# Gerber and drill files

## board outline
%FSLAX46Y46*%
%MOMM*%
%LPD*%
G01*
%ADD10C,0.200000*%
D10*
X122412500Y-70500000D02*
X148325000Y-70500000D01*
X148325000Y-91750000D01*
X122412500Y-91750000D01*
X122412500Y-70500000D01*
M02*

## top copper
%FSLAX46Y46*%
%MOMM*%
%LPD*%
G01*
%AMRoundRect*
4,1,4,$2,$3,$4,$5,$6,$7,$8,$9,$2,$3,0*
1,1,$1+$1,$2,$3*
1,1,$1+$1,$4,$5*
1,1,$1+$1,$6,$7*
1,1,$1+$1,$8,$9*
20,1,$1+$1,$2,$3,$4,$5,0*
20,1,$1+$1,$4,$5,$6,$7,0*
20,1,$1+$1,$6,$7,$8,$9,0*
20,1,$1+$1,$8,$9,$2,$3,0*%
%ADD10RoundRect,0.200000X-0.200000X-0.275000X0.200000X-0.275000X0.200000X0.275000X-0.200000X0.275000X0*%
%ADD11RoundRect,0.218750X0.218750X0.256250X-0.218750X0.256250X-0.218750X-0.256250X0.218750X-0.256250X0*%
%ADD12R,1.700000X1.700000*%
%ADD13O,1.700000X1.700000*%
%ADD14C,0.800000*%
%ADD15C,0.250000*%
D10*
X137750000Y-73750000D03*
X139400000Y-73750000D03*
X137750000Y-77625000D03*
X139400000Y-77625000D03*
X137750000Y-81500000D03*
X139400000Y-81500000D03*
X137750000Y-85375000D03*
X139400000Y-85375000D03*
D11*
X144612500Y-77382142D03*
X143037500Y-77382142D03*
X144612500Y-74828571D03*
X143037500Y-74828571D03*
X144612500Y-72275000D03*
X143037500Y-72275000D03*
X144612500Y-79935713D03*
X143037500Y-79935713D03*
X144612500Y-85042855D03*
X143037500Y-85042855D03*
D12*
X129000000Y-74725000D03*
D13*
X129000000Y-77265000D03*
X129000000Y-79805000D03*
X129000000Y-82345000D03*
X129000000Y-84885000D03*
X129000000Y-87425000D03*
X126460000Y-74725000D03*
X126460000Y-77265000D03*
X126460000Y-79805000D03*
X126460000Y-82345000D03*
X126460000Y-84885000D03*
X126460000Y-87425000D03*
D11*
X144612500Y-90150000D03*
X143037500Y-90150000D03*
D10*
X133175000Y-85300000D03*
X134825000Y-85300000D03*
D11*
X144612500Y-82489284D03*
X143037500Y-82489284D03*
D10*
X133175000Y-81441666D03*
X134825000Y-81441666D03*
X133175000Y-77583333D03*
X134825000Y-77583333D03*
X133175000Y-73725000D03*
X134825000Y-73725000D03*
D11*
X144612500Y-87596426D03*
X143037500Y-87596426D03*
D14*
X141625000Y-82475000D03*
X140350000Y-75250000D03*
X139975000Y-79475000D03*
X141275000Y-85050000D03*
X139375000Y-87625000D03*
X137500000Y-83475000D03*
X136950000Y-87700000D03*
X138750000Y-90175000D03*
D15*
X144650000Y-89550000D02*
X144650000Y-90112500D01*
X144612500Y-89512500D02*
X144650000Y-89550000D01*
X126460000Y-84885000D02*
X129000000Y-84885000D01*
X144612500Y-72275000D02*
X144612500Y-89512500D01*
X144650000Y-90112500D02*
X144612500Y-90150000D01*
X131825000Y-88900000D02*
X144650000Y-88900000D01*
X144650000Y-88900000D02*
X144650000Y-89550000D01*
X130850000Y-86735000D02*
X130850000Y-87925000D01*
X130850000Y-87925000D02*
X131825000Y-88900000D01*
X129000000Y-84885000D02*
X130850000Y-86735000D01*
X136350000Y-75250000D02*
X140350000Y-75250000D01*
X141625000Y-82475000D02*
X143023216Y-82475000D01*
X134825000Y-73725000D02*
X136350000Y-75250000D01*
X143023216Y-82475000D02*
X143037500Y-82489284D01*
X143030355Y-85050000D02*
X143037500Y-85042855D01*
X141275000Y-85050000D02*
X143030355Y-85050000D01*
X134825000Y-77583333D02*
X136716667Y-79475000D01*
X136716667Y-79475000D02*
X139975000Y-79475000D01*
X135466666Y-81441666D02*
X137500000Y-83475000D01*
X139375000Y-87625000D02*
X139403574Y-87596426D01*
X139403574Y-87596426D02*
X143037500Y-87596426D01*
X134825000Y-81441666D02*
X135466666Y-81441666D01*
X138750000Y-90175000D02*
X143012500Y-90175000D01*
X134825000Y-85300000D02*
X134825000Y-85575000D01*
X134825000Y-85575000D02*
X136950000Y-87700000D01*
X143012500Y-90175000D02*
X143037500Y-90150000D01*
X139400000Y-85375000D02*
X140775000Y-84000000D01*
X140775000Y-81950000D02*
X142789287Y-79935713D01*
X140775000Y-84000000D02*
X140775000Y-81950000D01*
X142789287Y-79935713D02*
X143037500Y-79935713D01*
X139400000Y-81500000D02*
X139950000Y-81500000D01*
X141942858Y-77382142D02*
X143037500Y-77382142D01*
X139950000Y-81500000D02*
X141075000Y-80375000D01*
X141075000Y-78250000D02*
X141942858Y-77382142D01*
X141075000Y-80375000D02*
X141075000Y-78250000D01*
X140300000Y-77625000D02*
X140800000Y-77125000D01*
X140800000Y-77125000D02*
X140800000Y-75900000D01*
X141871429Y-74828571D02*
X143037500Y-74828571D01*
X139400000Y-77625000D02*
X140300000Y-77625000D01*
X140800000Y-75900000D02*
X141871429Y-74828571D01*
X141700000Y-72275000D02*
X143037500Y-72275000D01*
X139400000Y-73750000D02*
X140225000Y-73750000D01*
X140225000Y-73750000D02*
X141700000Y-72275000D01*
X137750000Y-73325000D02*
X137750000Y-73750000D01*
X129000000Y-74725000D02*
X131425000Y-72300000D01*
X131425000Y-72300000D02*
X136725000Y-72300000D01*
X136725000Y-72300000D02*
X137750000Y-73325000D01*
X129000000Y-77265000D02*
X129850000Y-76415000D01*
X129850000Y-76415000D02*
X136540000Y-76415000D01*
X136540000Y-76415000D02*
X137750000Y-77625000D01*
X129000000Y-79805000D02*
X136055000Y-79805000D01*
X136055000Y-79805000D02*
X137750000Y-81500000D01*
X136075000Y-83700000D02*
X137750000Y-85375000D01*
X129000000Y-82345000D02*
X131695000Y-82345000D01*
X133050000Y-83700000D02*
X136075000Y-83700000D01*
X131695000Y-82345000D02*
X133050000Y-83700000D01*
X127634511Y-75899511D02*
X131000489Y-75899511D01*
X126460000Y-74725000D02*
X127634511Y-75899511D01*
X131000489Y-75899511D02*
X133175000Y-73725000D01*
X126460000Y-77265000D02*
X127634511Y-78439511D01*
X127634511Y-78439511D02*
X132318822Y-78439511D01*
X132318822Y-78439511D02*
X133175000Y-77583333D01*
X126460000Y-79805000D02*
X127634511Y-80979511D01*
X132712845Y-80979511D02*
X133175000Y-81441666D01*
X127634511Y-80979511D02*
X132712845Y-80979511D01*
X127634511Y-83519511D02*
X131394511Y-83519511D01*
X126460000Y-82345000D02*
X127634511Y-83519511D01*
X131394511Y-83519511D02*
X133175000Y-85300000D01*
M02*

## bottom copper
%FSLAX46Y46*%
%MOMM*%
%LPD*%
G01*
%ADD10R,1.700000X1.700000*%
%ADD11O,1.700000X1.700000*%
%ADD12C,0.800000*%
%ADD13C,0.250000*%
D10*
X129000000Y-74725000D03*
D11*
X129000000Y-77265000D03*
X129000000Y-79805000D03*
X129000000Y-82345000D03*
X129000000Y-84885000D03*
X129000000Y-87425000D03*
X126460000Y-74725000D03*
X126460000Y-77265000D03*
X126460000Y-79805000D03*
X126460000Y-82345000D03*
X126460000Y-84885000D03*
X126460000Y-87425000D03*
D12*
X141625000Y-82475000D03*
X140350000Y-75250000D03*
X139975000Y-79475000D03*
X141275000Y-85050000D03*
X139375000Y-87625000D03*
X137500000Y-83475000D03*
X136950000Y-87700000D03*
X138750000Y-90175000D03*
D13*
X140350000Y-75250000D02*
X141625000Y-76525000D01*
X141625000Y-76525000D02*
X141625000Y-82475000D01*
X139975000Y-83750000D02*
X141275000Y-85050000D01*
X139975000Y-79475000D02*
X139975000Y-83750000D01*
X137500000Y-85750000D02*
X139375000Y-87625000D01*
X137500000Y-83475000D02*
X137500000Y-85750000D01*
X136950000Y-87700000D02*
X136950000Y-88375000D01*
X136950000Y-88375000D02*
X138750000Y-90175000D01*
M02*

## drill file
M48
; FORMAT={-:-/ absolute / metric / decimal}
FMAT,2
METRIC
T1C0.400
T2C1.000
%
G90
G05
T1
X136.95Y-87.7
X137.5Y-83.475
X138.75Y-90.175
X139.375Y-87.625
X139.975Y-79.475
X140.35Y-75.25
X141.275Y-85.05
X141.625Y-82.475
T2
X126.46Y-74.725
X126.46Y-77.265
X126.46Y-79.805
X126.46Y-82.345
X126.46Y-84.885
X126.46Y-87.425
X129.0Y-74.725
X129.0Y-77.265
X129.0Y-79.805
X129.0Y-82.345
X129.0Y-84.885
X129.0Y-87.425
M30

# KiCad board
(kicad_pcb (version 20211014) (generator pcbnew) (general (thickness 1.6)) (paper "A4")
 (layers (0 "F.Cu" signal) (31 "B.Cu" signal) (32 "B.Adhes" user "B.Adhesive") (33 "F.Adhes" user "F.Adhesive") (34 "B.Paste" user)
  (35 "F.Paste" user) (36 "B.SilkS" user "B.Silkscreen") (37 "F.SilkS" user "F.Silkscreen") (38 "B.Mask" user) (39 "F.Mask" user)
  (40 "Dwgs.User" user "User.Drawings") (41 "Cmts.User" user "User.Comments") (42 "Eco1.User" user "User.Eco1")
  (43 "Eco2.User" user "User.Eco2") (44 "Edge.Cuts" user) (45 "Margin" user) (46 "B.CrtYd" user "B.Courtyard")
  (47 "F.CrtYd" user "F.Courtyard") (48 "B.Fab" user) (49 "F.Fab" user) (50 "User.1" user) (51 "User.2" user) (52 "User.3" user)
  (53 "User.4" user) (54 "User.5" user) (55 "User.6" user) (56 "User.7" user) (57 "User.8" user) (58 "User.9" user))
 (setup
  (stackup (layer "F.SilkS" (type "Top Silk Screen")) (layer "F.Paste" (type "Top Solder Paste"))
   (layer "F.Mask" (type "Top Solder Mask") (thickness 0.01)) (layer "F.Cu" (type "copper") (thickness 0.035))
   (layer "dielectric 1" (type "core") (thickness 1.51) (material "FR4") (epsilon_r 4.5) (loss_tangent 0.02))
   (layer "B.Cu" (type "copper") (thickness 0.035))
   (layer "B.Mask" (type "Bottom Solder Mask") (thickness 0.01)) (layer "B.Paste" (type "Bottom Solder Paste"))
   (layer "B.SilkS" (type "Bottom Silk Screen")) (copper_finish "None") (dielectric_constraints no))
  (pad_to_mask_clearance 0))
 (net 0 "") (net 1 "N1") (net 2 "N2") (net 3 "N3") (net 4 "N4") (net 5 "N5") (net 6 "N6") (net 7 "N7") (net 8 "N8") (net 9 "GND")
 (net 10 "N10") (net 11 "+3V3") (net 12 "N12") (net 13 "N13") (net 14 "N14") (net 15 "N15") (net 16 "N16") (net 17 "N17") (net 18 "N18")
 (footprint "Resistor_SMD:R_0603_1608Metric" (layer "F.Cu") (at 138.575 73.75)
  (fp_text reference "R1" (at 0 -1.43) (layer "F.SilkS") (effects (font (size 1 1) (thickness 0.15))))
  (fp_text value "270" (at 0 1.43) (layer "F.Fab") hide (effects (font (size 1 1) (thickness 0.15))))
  (pad "1" smd roundrect (at -0.825 0) (size 0.8 0.95) (layers "F.Cu" "F.Paste" "F.Mask") (roundrect_rratio 0.25) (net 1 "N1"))
  (pad "2" smd roundrect (at 0.825 0) (size 0.8 0.95) (layers "F.Cu" "F.Paste" "F.Mask") (roundrect_rratio 0.25) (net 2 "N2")))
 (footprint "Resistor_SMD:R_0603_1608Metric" (layer "F.Cu") (at 138.575 77.625)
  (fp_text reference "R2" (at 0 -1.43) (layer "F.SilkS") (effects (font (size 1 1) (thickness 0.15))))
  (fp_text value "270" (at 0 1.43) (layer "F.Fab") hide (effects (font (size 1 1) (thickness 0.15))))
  (pad "1" smd roundrect (at -0.825 0) (size 0.8 0.95) (layers "F.Cu" "F.Paste" "F.Mask") (roundrect_rratio 0.25) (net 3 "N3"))
  (pad "2" smd roundrect (at 0.825 0) (size 0.8 0.95) (layers "F.Cu" "F.Paste" "F.Mask") (roundrect_rratio 0.25) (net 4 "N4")))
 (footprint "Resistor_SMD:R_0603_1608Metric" (layer "F.Cu") (at 138.575 81.5)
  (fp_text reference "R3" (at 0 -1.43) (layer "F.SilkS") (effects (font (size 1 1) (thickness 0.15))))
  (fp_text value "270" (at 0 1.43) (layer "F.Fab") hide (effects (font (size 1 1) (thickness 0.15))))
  (pad "1" smd roundrect (at -0.825 0) (size 0.8 0.95) (layers "F.Cu" "F.Paste" "F.Mask") (roundrect_rratio 0.25) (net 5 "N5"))
  (pad "2" smd roundrect (at 0.825 0) (size 0.8 0.95) (layers "F.Cu" "F.Paste" "F.Mask") (roundrect_rratio 0.25) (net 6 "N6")))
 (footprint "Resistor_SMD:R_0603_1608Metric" (layer "F.Cu") (at 138.575 85.375)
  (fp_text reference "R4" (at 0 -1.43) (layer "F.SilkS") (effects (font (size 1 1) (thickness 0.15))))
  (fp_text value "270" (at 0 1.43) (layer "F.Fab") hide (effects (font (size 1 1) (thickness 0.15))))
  (pad "1" smd roundrect (at -0.825 0) (size 0.8 0.95) (layers "F.Cu" "F.Paste" "F.Mask") (roundrect_rratio 0.25) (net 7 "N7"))
  (pad "2" smd roundrect (at 0.825 0) (size 0.8 0.95) (layers "F.Cu" "F.Paste" "F.Mask") (roundrect_rratio 0.25) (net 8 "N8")))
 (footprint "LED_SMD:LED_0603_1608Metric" (layer "F.Cu") (at 143.825 77.382142 180)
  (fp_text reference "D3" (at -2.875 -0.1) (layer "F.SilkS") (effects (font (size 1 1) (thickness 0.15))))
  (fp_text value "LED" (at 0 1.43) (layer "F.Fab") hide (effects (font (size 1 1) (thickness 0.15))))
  (pad "1" smd roundrect (at -0.7875 0 180) (size 0.875 0.95) (layers "F.Cu" "F.Paste" "F.Mask") (roundrect_rratio 0.25) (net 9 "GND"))
  (pad "2" smd roundrect (at 0.7875 0 180) (size 0.875 0.95) (layers "F.Cu" "F.Paste" "F.Mask") (roundrect_rratio 0.25) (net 6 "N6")))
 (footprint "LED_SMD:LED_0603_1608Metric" (layer "F.Cu") (at 143.825 74.828571 180)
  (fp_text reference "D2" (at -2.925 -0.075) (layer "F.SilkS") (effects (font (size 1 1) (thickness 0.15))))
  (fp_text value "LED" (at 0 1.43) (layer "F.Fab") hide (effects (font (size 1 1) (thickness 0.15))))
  (pad "1" smd roundrect (at -0.7875 0 180) (size 0.875 0.95) (layers "F.Cu" "F.Paste" "F.Mask") (roundrect_rratio 0.25) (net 9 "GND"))
  (pad "2" smd roundrect (at 0.7875 0 180) (size 0.875 0.95) (layers "F.Cu" "F.Paste" "F.Mask") (roundrect_rratio 0.25) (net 4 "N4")))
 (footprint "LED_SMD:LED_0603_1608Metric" (layer "F.Cu") (at 143.825 72.275 180)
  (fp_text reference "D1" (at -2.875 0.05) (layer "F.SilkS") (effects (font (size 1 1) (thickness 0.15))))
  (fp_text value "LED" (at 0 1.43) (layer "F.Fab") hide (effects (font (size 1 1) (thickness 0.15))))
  (pad "1" smd roundrect (at -0.7875 0 180) (size 0.875 0.95) (layers "F.Cu" "F.Paste" "F.Mask") (roundrect_rratio 0.25) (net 9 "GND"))
  (pad "2" smd roundrect (at 0.7875 0 180) (size 0.875 0.95) (layers "F.Cu" "F.Paste" "F.Mask") (roundrect_rratio 0.25) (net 2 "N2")))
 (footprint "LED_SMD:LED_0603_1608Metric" (layer "F.Cu") (at 143.825 79.935713 180)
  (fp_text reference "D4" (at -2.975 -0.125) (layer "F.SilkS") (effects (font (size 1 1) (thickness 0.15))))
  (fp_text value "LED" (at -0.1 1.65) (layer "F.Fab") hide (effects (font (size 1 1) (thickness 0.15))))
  (pad "1" smd roundrect (at -0.7875 0 180) (size 0.875 0.95) (layers "F.Cu" "F.Paste" "F.Mask") (roundrect_rratio 0.25) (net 9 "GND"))
  (pad "2" smd roundrect (at 0.7875 0 180) (size 0.875 0.95) (layers "F.Cu" "F.Paste" "F.Mask") (roundrect_rratio 0.25) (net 8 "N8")))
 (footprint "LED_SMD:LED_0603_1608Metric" (layer "F.Cu") (at 143.825 85.042855 180)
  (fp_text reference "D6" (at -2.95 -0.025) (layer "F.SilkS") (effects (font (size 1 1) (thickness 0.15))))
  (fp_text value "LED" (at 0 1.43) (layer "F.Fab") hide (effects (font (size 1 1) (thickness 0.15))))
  (pad "1" smd roundrect (at -0.7875 0 180) (size 0.875 0.95) (layers "F.Cu" "F.Paste" "F.Mask") (roundrect_rratio 0.25) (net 9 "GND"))
  (pad "2" smd roundrect (at 0.7875 0 180) (size 0.875 0.95) (layers "F.Cu" "F.Paste" "F.Mask") (roundrect_rratio 0.25) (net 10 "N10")))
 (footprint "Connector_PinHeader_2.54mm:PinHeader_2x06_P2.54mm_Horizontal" (layer "F.Cu") (at 129 87.425 180)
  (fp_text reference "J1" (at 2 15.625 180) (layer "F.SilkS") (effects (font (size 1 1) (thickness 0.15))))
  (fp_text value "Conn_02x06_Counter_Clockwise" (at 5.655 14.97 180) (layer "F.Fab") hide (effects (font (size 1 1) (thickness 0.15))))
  (pad "1" thru_hole rect (at 0 12.7 180) (size 1.7 1.7) (drill 1) (layers *.Cu *.Mask) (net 1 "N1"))
  (pad "2" thru_hole oval (at 0 10.16 180) (size 1.7 1.7) (drill 1) (layers *.Cu *.Mask) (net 3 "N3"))
  (pad "3" thru_hole oval (at 0 7.62 180) (size 1.7 1.7) (drill 1) (layers *.Cu *.Mask) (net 5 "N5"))
  (pad "4" thru_hole oval (at 0 5.08 180) (size 1.7 1.7) (drill 1) (layers *.Cu *.Mask) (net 7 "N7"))
  (pad "5" thru_hole oval (at 0 2.54 180) (size 1.7 1.7) (drill 1) (layers *.Cu *.Mask) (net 9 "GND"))
  (pad "6" thru_hole oval (at 0 0 180) (size 1.7 1.7) (drill 1) (layers *.Cu *.Mask) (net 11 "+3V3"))
  (pad "7" thru_hole oval (at 2.54 12.7 180) (size 1.7 1.7) (drill 1) (layers *.Cu *.Mask) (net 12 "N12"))
  (pad "8" thru_hole oval (at 2.54 10.16 180) (size 1.7 1.7) (drill 1) (layers *.Cu *.Mask) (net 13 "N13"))
  (pad "9" thru_hole oval (at 2.54 7.62 180) (size 1.7 1.7) (drill 1) (layers *.Cu *.Mask) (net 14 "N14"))
  (pad "10" thru_hole oval (at 2.54 5.08 180) (size 1.7 1.7) (drill 1) (layers *.Cu *.Mask) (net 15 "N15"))
  (pad "11" thru_hole oval (at 2.54 2.54 180) (size 1.7 1.7) (drill 1) (layers *.Cu *.Mask) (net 9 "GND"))
  (pad "12" thru_hole oval (at 2.54 0 180) (size 1.7 1.7) (drill 1) (layers *.Cu *.Mask) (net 11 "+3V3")))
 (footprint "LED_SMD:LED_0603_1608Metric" (layer "F.Cu") (at 143.825 90.15 180)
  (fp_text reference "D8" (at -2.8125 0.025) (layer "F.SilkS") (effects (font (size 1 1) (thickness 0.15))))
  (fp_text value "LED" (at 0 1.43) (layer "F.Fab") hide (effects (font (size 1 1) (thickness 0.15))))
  (pad "1" smd roundrect (at -0.7875 0 180) (size 0.875 0.95) (layers "F.Cu" "F.Paste" "F.Mask") (roundrect_rratio 0.25) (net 9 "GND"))
  (pad "2" smd roundrect (at 0.7875 0 180) (size 0.875 0.95) (layers "F.Cu" "F.Paste" "F.Mask") (roundrect_rratio 0.25) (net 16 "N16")))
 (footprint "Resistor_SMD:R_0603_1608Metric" (layer "F.Cu") (at 134 85.3)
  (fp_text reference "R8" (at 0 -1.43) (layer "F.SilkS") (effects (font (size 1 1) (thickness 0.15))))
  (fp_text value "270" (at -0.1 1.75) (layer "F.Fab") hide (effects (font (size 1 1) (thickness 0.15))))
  (pad "1" smd roundrect (at -0.825 0) (size 0.8 0.95) (layers "F.Cu" "F.Paste" "F.Mask") (roundrect_rratio 0.25) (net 15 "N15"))
  (pad "2" smd roundrect (at 0.825 0) (size 0.8 0.95) (layers "F.Cu" "F.Paste" "F.Mask") (roundrect_rratio 0.25) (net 16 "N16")))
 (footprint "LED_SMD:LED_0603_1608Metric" (layer "F.Cu") (at 143.825 82.489284 180)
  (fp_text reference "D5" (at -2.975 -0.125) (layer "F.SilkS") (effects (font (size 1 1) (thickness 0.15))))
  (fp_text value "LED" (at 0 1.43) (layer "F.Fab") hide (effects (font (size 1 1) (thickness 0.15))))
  (pad "1" smd roundrect (at -0.7875 0 180) (size 0.875 0.95) (layers "F.Cu" "F.Paste" "F.Mask") (roundrect_rratio 0.25) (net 9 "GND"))
  (pad "2" smd roundrect (at 0.7875 0 180) (size 0.875 0.95) (layers "F.Cu" "F.Paste" "F.Mask") (roundrect_rratio 0.25) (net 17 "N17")))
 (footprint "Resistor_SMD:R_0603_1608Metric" (layer "F.Cu") (at 134 81.441666)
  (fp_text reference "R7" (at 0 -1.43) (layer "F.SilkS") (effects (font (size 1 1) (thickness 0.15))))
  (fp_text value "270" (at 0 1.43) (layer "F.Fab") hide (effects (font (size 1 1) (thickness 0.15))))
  (pad "1" smd roundrect (at -0.825 0) (size 0.8 0.95) (layers "F.Cu" "F.Paste" "F.Mask") (roundrect_rratio 0.25) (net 14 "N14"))
  (pad "2" smd roundrect (at 0.825 0) (size 0.8 0.95) (layers "F.Cu" "F.Paste" "F.Mask") (roundrect_rratio 0.25) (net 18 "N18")))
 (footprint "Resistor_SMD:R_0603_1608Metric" (layer "F.Cu") (at 134 77.583333)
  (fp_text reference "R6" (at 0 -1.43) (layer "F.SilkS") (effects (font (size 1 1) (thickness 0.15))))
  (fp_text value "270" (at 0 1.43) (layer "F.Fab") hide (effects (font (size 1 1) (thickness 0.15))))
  (pad "1" smd roundrect (at -0.825 0) (size 0.8 0.95) (layers "F.Cu" "F.Paste" "F.Mask") (roundrect_rratio 0.25) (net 13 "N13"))
  (pad "2" smd roundrect (at 0.825 0) (size 0.8 0.95) (layers "F.Cu" "F.Paste" "F.Mask") (roundrect_rratio 0.25) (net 10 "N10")))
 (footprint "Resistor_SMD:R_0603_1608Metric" (layer "F.Cu") (at 134 73.725)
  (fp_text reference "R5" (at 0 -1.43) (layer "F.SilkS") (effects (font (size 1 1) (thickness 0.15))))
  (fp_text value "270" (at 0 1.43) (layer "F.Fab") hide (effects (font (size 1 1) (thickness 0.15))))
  (pad "1" smd roundrect (at -0.825 0) (size 0.8 0.95) (layers "F.Cu" "F.Paste" "F.Mask") (roundrect_rratio 0.25) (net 12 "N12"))
  (pad "2" smd roundrect (at 0.825 0) (size 0.8 0.95) (layers "F.Cu" "F.Paste" "F.Mask") (roundrect_rratio 0.25) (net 17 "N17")))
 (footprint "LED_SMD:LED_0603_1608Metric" (layer "F.Cu") (at 143.825 87.596426 180)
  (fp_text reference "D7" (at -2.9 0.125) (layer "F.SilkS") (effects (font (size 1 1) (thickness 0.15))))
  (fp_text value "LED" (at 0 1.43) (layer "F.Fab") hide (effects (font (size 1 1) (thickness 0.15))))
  (pad "1" smd roundrect (at -0.7875 0 180) (size 0.875 0.95) (layers "F.Cu" "F.Paste" "F.Mask") (roundrect_rratio 0.25) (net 9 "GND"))
  (pad "2" smd roundrect (at 0.7875 0 180) (size 0.875 0.95) (layers "F.Cu" "F.Paste" "F.Mask") (roundrect_rratio 0.25) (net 18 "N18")))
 (gr_rect (start 122.4125 70.5) (end 148.325 91.75) (layer "Edge.Cuts") (width 0.2) (fill none))
 (segment (start 144.65 89.55) (end 144.65 90.1125) (width 0.25) (layer "F.Cu") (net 9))
 (segment (start 144.6125 89.5125) (end 144.65 89.55) (width 0.25) (layer "F.Cu") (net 9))
 (segment (start 126.46 84.885) (end 129 84.885) (width 0.25) (layer "F.Cu") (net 9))
 (segment (start 144.6125 72.275) (end 144.6125 89.5125) (width 0.25) (layer "F.Cu") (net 9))
 (segment (start 144.65 90.1125) (end 144.6125 90.15) (width 0.25) (layer "F.Cu") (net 9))
 (segment (start 131.825 88.9) (end 144.65 88.9) (width 0.25) (layer "F.Cu") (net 9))
 (segment (start 144.65 88.9) (end 144.65 89.55) (width 0.25) (layer "F.Cu") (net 9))
 (segment (start 130.85 86.735) (end 130.85 87.925) (width 0.25) (layer "F.Cu") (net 9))
 (segment (start 130.85 87.925) (end 131.825 88.9) (width 0.25) (layer "F.Cu") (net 9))
 (segment (start 129 84.885) (end 130.85 86.735) (width 0.25) (layer "F.Cu") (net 9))
 (segment (start 136.35 75.25) (end 140.35 75.25) (width 0.25) (layer "F.Cu") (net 17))
 (segment (start 141.625 82.475) (end 143.023216 82.475) (width 0.25) (layer "F.Cu") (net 17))
 (segment (start 134.825 73.725) (end 136.35 75.25) (width 0.25) (layer "F.Cu") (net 17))
 (segment (start 143.023216 82.475) (end 143.0375 82.489284) (width 0.25) (layer "F.Cu") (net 17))
 (via (at 141.625 82.475) (size 0.8) (drill 0.4) (layers "F.Cu" "B.Cu") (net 17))
 (via (at 140.35 75.25) (size 0.8) (drill 0.4) (layers "F.Cu" "B.Cu") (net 17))
 (segment (start 140.35 75.25) (end 141.625 76.525) (width 0.25) (layer "B.Cu") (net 17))
 (segment (start 141.625 76.525) (end 141.625 82.475) (width 0.25) (layer "B.Cu") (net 17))
 (segment (start 143.030355 85.05) (end 143.0375 85.042855) (width 0.25) (layer "F.Cu") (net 10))
 (segment (start 141.275 85.05) (end 143.030355 85.05) (width 0.25) (layer "F.Cu") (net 10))
 (segment (start 134.825 77.583333) (end 136.716667 79.475) (width 0.25) (layer "F.Cu") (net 10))
 (segment (start 136.716667 79.475) (end 139.975 79.475) (width 0.25) (layer "F.Cu") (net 10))
 (via (at 139.975 79.475) (size 0.8) (drill 0.4) (layers "F.Cu" "B.Cu") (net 10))
 (via (at 141.275 85.05) (size 0.8) (drill 0.4) (layers "F.Cu" "B.Cu") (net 10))
 (segment (start 139.975 83.75) (end 141.275 85.05) (width 0.25) (layer "B.Cu") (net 10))
 (segment (start 139.975 79.475) (end 139.975 83.75) (width 0.25) (layer "B.Cu") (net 10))
 (segment (start 135.466666 81.441666) (end 137.5 83.475) (width 0.25) (layer "F.Cu") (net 18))
 (segment (start 139.375 87.625) (end 139.403574 87.596426) (width 0.25) (layer "F.Cu") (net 18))
 (segment (start 139.403574 87.596426) (end 143.0375 87.596426) (width 0.25) (layer "F.Cu") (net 18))
 (segment (start 134.825 81.441666) (end 135.466666 81.441666) (width 0.25) (layer "F.Cu") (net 18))
 (via (at 139.375 87.625) (size 0.8) (drill 0.4) (layers "F.Cu" "B.Cu") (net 18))
 (via (at 137.5 83.475) (size 0.8) (drill 0.4) (layers "F.Cu" "B.Cu") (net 18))
 (segment (start 137.5 85.75) (end 139.375 87.625) (width 0.25) (layer "B.Cu") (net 18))
 (segment (start 137.5 83.475) (end 137.5 85.75) (width 0.25) (layer "B.Cu") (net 18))
 (segment (start 138.75 90.175) (end 143.0125 90.175) (width 0.25) (layer "F.Cu") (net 16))
 (segment (start 134.825 85.3) (end 134.825 85.575) (width 0.25) (layer "F.Cu") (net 16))
 (segment (start 134.825 85.575) (end 136.95 87.7) (width 0.25) (layer "F.Cu") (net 16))
 (segment (start 143.0125 90.175) (end 143.0375 90.15) (width 0.25) (layer "F.Cu") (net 16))
 (via (at 136.95 87.7) (size 0.8) (drill 0.4) (layers "F.Cu" "B.Cu") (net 16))
 (via (at 138.75 90.175) (size 0.8) (drill 0.4) (layers "F.Cu" "B.Cu") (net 16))
 (segment (start 136.95 87.7) (end 136.95 88.375) (width 0.25) (layer "B.Cu") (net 16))
 (segment (start 136.95 88.375) (end 138.75 90.175) (width 0.25) (layer "B.Cu") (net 16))
 (segment (start 139.4 85.375) (end 140.775 84) (width 0.25) (layer "F.Cu") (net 8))
 (segment (start 140.775 81.95) (end 142.789287 79.935713) (width 0.25) (layer "F.Cu") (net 8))
 (segment (start 140.775 84) (end 140.775 81.95) (width 0.25) (layer "F.Cu") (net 8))
 (segment (start 142.789287 79.935713) (end 143.0375 79.935713) (width 0.25) (layer "F.Cu") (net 8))
 (segment (start 139.4 81.5) (end 139.95 81.5) (width 0.25) (layer "F.Cu") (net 6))
 (segment (start 141.942858 77.382142) (end 143.0375 77.382142) (width 0.25) (layer "F.Cu") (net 6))
 (segment (start 139.95 81.5) (end 141.075 80.375) (width 0.25) (layer "F.Cu") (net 6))
 (segment (start 141.075 78.25) (end 141.942858 77.382142) (width 0.25) (layer "F.Cu") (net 6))
 (segment (start 141.075 80.375) (end 141.075 78.25) (width 0.25) (layer "F.Cu") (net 6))
 (segment (start 140.3 77.625) (end 140.8 77.125) (width 0.25) (layer "F.Cu") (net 4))
 (segment (start 140.8 77.125) (end 140.8 75.9) (width 0.25) (layer "F.Cu") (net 4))
 (segment (start 141.871429 74.828571) (end 143.0375 74.828571) (width 0.25) (layer "F.Cu") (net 4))
 (segment (start 139.4 77.625) (end 140.3 77.625) (width 0.25) (layer "F.Cu") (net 4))
 (segment (start 140.8 75.9) (end 141.871429 74.828571) (width 0.25) (layer "F.Cu") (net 4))
 (segment (start 141.7 72.275) (end 143.0375 72.275) (width 0.25) (layer "F.Cu") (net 2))
 (segment (start 139.4 73.75) (end 140.225 73.75) (width 0.25) (layer "F.Cu") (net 2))
 (segment (start 140.225 73.75) (end 141.7 72.275) (width 0.25) (layer "F.Cu") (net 2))
 (segment (start 137.75 73.325) (end 137.75 73.75) (width 0.25) (layer "F.Cu") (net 1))
 (segment (start 129 74.725) (end 131.425 72.3) (width 0.25) (layer "F.Cu") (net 1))
 (segment (start 131.425 72.3) (end 136.725 72.3) (width 0.25) (layer "F.Cu") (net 1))
 (segment (start 136.725 72.3) (end 137.75 73.325) (width 0.25) (layer "F.Cu") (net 1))
 (segment (start 129 77.265) (end 129.85 76.415) (width 0.25) (layer "F.Cu") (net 3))
 (segment (start 129.85 76.415) (end 136.54 76.415) (width 0.25) (layer "F.Cu") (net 3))
 (segment (start 136.54 76.415) (end 137.75 77.625) (width 0.25) (layer "F.Cu") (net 3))
 (segment (start 129 79.805) (end 136.055 79.805) (width 0.25) (layer "F.Cu") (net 5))
 (segment (start 136.055 79.805) (end 137.75 81.5) (width 0.25) (layer "F.Cu") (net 5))
 (segment (start 136.075 83.7) (end 137.75 85.375) (width 0.25) (layer "F.Cu") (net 7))
 (segment (start 129 82.345) (end 131.695 82.345) (width 0.25) (layer "F.Cu") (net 7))
 (segment (start 133.05 83.7) (end 136.075 83.7) (width 0.25) (layer "F.Cu") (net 7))
 (segment (start 131.695 82.345) (end 133.05 83.7) (width 0.25) (layer "F.Cu") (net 7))
 (segment (start 127.634511 75.899511) (end 131.000489 75.899511) (width 0.25) (layer "F.Cu") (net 12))
 (segment (start 126.46 74.725) (end 127.634511 75.899511) (width 0.25) (layer "F.Cu") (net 12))
 (segment (start 131.000489 75.899511) (end 133.175 73.725) (width 0.25) (layer "F.Cu") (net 12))
 (segment (start 126.46 77.265) (end 127.634511 78.439511) (width 0.25) (layer "F.Cu") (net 13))
 (segment (start 127.634511 78.439511) (end 132.318822 78.439511) (width 0.25) (layer "F.Cu") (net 13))
 (segment (start 132.318822 78.439511) (end 133.175 77.583333) (width 0.25) (layer "F.Cu") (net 13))
 (segment (start 126.46 79.805) (end 127.634511 80.979511) (width 0.25) (layer "F.Cu") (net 14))
 (segment (start 132.712845 80.979511) (end 133.175 81.441666) (width 0.25) (layer "F.Cu") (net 14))
 (segment (start 127.634511 80.979511) (end 132.712845 80.979511) (width 0.25) (layer "F.Cu") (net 14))
 (segment (start 127.634511 83.519511) (end 131.394511 83.519511) (width 0.25) (layer "F.Cu") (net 15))
 (segment (start 126.46 82.345) (end 127.634511 83.519511) (width 0.25) (layer "F.Cu") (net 15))
 (segment (start 131.394511 83.519511) (end 133.175 85.3) (width 0.25) (layer "F.Cu") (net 15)))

